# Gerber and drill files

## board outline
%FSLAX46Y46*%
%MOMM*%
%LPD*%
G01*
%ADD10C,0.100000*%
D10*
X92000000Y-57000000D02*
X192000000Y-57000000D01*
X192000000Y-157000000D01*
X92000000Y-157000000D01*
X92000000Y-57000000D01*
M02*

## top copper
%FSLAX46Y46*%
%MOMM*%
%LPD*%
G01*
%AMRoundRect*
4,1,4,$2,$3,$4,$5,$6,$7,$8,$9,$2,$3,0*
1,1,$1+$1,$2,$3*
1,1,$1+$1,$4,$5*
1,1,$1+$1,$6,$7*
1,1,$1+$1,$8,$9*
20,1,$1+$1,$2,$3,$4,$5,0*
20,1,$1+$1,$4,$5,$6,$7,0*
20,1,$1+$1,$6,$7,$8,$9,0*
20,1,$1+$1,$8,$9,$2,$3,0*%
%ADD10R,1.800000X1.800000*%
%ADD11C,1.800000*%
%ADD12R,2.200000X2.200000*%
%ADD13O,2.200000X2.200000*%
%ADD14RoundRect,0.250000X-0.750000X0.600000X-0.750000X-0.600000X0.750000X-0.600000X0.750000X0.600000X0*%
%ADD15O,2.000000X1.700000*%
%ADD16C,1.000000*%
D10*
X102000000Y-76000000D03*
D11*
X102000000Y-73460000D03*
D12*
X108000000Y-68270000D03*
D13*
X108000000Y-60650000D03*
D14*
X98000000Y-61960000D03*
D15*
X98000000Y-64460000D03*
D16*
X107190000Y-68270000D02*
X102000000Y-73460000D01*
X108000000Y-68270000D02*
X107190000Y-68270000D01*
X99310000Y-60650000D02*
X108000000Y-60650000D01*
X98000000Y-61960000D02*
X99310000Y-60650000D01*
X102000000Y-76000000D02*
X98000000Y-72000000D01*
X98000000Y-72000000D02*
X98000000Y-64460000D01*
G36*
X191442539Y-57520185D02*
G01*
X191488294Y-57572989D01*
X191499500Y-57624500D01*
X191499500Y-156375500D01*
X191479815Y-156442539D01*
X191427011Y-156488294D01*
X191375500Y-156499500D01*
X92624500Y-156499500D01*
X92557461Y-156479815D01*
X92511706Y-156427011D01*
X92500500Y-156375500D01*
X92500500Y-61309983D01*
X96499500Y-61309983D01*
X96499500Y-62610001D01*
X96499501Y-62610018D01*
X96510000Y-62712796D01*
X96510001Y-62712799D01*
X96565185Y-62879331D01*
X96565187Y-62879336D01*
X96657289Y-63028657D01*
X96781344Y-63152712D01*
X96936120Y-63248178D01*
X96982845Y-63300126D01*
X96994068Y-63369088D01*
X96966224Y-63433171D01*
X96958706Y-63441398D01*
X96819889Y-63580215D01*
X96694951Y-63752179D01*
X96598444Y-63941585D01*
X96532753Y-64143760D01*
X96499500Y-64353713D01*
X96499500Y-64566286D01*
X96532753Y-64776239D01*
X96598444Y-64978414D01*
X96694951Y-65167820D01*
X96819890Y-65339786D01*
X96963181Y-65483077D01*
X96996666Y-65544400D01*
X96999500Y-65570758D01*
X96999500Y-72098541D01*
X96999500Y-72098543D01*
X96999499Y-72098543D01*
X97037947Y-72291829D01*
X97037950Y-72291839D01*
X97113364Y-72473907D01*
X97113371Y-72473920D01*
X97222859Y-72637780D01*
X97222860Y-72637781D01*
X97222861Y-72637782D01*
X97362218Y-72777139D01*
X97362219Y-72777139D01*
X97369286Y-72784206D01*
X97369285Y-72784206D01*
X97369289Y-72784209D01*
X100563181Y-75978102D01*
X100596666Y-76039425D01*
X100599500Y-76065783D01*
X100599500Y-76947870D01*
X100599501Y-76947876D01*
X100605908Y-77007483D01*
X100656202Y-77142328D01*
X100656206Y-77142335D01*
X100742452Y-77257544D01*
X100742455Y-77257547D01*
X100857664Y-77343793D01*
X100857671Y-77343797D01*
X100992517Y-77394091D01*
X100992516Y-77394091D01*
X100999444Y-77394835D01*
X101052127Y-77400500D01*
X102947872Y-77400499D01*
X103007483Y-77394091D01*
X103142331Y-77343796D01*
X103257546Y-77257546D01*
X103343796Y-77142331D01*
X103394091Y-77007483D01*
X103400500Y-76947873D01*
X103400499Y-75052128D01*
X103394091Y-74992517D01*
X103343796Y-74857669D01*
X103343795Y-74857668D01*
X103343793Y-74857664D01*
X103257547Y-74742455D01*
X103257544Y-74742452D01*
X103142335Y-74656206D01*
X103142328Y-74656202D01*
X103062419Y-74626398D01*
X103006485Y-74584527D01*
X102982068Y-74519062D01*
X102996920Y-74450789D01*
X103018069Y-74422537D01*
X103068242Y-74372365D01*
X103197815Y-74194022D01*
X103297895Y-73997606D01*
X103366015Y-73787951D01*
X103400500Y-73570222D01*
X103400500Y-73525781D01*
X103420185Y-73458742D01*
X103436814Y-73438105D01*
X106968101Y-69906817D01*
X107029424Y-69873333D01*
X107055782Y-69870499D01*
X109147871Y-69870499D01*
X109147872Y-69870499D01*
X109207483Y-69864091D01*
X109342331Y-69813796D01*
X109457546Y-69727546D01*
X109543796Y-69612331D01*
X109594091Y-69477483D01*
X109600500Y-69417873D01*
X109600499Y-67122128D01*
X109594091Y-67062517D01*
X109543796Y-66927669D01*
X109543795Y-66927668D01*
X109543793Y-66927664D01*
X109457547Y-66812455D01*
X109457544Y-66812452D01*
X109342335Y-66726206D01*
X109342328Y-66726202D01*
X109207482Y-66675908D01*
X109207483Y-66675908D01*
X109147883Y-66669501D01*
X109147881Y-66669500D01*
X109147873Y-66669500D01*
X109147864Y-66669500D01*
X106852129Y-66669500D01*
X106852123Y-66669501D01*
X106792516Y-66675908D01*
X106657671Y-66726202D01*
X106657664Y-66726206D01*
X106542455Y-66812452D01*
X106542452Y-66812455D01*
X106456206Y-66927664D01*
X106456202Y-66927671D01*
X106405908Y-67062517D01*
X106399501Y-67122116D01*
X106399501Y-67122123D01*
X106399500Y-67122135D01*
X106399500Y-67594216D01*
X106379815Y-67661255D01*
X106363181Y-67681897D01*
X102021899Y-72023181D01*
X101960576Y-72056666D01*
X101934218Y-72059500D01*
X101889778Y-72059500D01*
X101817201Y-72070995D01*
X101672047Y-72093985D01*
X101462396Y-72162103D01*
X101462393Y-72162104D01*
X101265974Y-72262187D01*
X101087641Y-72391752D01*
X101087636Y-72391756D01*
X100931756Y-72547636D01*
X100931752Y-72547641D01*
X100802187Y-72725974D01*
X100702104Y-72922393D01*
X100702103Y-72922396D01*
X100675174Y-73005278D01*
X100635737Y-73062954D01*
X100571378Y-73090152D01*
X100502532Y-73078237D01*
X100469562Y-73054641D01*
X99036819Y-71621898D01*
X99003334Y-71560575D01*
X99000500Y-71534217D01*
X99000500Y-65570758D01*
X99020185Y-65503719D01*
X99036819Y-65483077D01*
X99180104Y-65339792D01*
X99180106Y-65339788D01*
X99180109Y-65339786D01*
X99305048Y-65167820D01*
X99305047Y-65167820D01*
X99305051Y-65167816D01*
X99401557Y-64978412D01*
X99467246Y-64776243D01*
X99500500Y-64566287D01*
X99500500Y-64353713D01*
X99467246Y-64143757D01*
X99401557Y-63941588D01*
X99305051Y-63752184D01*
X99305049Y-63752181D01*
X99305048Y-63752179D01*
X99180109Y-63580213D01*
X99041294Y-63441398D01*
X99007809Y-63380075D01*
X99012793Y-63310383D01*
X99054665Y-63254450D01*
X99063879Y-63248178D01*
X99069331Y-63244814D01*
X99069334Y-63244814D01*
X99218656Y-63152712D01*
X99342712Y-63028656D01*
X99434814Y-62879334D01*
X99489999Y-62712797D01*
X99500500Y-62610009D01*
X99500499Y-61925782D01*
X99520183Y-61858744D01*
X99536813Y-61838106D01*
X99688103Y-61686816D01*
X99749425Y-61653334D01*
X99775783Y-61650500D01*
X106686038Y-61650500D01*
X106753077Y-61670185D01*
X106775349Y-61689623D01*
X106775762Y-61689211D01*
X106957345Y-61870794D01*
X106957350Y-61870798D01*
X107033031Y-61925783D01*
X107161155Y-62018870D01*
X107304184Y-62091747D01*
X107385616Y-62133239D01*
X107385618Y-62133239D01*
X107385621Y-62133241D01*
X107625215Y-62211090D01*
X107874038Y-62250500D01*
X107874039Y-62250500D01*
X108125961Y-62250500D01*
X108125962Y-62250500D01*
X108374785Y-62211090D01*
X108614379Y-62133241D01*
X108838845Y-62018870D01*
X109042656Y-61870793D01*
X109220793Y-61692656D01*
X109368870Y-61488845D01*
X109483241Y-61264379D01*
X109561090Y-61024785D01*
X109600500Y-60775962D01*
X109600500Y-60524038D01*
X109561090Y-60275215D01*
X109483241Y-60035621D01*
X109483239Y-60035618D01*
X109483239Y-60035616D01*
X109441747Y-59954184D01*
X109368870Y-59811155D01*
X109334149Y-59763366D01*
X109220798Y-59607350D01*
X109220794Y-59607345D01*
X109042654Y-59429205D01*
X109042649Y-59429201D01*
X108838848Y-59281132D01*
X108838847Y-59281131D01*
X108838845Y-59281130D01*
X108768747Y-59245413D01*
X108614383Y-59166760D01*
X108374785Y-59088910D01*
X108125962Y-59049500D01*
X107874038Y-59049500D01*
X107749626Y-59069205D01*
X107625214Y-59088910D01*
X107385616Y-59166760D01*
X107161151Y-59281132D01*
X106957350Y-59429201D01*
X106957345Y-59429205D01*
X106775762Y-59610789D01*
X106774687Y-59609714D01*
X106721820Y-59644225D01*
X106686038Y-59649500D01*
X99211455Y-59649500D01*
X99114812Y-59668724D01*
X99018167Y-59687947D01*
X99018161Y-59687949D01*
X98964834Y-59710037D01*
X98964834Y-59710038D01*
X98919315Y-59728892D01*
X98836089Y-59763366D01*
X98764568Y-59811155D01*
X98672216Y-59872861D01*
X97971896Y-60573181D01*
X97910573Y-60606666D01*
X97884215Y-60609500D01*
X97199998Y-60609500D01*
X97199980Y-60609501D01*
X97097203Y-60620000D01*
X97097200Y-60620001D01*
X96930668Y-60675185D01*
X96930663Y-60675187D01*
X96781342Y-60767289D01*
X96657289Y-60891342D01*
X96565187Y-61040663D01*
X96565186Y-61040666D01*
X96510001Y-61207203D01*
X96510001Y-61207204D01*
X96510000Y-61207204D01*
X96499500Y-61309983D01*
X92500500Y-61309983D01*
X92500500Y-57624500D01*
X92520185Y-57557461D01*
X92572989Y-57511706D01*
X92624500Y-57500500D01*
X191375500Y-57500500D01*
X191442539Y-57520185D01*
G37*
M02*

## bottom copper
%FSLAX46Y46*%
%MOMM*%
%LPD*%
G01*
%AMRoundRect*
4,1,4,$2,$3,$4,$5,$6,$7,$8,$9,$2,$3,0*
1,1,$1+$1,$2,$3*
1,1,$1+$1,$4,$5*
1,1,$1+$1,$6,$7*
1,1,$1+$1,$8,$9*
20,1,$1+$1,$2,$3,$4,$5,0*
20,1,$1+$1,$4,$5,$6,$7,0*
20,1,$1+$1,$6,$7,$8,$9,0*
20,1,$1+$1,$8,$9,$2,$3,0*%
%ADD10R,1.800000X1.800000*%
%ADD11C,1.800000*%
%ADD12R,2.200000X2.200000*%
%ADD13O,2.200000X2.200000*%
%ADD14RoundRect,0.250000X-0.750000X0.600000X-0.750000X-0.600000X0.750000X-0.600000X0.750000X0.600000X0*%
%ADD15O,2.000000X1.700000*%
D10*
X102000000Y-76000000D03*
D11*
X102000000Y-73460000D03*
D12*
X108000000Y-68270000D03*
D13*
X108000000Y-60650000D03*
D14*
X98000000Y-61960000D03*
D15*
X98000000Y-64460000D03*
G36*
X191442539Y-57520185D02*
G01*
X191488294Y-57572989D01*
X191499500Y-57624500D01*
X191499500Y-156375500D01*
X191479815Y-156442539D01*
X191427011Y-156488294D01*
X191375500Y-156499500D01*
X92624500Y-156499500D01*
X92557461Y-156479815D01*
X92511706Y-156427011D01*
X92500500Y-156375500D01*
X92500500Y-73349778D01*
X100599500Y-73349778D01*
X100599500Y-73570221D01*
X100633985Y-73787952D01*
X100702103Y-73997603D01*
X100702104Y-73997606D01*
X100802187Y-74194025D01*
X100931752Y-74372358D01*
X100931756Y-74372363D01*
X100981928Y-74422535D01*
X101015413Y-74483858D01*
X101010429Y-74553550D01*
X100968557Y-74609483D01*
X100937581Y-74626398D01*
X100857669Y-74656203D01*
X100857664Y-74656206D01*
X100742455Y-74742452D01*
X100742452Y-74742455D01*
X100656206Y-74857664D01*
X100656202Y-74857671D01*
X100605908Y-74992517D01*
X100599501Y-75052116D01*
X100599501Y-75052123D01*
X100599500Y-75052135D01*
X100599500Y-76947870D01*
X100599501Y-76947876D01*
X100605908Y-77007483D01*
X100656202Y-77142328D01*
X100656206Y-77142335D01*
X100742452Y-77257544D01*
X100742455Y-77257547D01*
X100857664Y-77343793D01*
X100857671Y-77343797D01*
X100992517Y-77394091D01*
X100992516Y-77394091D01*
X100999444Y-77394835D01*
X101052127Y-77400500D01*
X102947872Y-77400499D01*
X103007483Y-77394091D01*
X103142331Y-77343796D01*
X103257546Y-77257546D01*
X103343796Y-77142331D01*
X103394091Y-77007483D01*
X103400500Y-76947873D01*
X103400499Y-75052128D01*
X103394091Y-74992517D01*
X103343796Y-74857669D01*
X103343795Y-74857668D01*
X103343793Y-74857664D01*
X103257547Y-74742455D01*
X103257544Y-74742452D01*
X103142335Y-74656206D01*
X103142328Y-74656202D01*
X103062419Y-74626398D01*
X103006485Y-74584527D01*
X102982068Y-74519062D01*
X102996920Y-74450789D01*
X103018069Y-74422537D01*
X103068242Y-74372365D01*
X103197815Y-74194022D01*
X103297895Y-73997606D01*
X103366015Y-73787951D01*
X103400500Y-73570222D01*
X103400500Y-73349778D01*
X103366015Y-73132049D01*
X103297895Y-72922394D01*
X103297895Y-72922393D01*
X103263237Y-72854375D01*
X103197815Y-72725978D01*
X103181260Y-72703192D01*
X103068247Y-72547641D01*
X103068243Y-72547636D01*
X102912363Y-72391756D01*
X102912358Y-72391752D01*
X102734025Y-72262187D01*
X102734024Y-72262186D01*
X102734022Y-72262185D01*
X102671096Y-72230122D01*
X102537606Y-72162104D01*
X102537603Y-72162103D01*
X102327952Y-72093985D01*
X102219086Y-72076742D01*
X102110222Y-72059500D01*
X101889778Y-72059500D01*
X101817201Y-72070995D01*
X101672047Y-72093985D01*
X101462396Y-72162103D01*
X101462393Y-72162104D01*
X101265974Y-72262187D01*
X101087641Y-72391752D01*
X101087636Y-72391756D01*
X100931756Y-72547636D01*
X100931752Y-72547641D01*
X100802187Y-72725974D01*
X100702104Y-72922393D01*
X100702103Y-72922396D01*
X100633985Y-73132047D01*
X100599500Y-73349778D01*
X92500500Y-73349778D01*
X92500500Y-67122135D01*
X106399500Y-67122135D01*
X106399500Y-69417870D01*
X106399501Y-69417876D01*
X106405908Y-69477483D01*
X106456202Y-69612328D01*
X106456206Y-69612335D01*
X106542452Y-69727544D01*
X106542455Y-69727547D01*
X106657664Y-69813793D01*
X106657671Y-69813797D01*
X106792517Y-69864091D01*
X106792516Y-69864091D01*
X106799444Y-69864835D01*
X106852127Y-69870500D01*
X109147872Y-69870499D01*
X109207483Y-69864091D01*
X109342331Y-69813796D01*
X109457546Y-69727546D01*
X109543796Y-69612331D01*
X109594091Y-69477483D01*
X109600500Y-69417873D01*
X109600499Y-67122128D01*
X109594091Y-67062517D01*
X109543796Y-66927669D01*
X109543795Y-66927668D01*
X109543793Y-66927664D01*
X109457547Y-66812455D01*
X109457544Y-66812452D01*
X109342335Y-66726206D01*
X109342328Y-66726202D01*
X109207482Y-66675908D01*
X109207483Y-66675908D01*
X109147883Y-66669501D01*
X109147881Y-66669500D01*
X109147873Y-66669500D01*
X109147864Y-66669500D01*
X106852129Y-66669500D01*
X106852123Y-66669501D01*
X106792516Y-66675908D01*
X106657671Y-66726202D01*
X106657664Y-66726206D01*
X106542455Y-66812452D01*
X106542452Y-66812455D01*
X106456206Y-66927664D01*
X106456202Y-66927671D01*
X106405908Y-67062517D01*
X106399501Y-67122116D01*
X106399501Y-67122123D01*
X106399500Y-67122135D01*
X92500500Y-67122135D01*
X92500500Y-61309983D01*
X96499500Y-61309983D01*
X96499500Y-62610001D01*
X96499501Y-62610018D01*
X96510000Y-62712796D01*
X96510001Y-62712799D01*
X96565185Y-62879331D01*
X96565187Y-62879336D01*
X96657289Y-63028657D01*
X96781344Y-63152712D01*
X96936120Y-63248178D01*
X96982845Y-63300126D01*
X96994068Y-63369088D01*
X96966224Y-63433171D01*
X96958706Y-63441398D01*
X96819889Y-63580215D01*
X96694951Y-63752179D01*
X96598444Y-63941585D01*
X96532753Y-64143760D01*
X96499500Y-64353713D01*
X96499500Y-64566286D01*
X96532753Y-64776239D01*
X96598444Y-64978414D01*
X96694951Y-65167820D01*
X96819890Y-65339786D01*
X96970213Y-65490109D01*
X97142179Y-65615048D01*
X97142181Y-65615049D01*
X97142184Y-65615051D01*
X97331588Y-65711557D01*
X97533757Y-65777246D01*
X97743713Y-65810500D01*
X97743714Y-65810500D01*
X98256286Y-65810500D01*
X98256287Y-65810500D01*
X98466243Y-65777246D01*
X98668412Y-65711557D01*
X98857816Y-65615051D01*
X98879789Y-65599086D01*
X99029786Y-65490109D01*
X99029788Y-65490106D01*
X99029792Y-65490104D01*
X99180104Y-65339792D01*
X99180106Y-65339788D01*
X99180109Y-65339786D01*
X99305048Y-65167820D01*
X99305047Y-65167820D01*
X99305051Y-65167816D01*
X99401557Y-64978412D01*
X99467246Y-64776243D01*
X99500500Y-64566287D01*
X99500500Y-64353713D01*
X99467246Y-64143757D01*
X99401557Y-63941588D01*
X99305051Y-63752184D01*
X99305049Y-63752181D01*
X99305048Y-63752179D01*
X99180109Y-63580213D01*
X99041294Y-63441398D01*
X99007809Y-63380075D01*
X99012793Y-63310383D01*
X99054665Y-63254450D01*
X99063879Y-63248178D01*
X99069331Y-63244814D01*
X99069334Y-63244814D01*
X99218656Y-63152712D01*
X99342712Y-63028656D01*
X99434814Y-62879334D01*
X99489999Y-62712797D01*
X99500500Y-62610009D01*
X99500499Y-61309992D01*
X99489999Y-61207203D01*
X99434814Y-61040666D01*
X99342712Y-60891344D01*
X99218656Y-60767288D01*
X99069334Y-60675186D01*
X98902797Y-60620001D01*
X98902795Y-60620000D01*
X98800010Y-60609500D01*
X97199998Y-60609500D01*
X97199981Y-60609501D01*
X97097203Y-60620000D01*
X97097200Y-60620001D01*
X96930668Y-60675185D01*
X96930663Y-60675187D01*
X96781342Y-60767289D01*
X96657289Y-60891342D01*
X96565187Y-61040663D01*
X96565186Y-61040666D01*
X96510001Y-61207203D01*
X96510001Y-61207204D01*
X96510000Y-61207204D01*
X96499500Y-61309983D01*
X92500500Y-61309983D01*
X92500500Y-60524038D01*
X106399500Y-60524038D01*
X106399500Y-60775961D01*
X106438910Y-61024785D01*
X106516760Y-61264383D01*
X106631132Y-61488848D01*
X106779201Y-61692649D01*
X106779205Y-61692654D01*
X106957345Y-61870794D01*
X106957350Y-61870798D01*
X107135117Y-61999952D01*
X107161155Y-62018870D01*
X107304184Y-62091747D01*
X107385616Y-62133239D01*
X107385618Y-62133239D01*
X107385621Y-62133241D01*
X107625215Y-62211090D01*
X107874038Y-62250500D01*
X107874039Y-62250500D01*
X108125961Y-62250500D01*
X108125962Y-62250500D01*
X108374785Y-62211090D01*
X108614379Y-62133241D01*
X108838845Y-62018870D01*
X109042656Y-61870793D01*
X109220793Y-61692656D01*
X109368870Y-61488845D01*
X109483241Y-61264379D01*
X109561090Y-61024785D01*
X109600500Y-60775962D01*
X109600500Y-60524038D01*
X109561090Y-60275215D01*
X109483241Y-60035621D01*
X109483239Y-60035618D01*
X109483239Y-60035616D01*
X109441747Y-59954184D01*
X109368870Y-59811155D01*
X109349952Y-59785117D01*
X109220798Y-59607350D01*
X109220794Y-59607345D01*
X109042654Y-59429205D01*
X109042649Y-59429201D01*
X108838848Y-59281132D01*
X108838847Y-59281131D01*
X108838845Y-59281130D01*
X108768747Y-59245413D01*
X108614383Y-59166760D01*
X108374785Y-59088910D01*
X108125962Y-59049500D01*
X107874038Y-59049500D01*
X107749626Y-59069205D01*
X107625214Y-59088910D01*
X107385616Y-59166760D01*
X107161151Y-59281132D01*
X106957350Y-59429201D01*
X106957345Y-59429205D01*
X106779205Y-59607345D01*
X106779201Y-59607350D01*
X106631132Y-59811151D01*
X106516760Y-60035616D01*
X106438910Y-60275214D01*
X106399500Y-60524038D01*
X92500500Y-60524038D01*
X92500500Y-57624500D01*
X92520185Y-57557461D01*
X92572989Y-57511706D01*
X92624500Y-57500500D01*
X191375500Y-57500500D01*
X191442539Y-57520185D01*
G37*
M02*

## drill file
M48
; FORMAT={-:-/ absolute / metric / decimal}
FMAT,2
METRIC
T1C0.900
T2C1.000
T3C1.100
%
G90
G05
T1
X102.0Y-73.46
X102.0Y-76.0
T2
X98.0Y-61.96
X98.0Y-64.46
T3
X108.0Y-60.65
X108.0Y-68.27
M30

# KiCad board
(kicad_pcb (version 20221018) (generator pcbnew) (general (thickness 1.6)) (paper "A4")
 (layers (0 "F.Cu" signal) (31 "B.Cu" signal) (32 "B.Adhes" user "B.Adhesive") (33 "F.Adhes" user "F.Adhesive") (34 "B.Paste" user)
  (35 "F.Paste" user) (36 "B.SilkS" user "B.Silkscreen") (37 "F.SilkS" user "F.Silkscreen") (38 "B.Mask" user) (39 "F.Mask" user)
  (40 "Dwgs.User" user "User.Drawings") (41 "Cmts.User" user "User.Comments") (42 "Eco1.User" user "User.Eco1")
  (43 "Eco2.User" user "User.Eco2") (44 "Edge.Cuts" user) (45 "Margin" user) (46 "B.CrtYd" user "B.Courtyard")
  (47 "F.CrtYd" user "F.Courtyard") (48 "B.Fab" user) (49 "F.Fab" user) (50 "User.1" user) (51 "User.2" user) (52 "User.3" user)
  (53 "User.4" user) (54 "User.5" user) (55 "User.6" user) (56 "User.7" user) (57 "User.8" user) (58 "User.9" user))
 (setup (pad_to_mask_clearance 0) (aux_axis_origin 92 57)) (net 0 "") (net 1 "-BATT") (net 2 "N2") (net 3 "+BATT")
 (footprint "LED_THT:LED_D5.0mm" (layer "F.Cu") (at 102 76 90)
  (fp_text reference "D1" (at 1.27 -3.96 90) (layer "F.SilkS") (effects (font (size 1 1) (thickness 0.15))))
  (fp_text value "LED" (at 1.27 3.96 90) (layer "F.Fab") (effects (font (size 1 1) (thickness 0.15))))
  (pad "1" thru_hole rect (at 0 0 90) (size 1.8 1.8) (drill 0.9) (layers "*.Cu" "*.Mask") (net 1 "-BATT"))
  (pad "2" thru_hole circle (at 2.54 0 90) (size 1.8 1.8) (drill 0.9) (layers "*.Cu" "*.Mask") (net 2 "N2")))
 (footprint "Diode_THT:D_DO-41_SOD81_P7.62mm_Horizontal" (layer "F.Cu") (at 108 68.27 90)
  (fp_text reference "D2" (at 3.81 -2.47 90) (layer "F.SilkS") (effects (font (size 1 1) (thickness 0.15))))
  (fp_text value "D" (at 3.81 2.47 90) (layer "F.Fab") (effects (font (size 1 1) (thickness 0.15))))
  (pad "1" thru_hole rect (at 0 0 90) (size 2.2 2.2) (drill 1.1) (layers "*.Cu" "*.Mask") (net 2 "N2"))
  (pad "2" thru_hole oval (at 7.62 0 90) (size 2.2 2.2) (drill 1.1) (layers "*.Cu" "*.Mask") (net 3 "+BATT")))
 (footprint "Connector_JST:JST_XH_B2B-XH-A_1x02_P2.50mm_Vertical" (layer "F.Cu") (at 98 61.96 -90)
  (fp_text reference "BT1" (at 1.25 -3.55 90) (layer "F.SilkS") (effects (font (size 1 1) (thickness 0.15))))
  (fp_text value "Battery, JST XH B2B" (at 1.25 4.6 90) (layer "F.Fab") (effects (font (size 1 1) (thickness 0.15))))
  (pad "1" thru_hole roundrect (at 0 0 270) (size 1.7 2) (drill 1) (layers "*.Cu" "*.Mask") (roundrect_rratio 0.147059) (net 3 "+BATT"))
  (pad "2" thru_hole oval (at 2.5 0 270) (size 1.7 2) (drill 1) (layers "*.Cu" "*.Mask") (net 1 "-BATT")))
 (gr_rect (start 92 57) (end 192 157) (stroke (width 0.1) (type default)) (fill none) (layer "Edge.Cuts"))
 (segment (start 107.19 68.27) (end 102 73.46) (width 1) (layer "F.Cu") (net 2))
 (segment (start 108 68.27) (end 107.19 68.27) (width 1) (layer "F.Cu") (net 2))
 (segment (start 99.31 60.65) (end 108 60.65) (width 1) (layer "F.Cu") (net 3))
 (segment (start 98 61.96) (end 99.31 60.65) (width 1) (layer "F.Cu") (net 3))
 (segment (start 102 76) (end 98 72) (width 1) (layer "F.Cu") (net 1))
 (segment (start 98 72) (end 98 64.46) (width 1) (layer "F.Cu") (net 1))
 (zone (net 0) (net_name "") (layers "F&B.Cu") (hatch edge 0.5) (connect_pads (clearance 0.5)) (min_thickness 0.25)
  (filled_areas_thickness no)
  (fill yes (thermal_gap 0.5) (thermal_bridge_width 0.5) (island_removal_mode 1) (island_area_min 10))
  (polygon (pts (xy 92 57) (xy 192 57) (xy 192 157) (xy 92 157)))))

